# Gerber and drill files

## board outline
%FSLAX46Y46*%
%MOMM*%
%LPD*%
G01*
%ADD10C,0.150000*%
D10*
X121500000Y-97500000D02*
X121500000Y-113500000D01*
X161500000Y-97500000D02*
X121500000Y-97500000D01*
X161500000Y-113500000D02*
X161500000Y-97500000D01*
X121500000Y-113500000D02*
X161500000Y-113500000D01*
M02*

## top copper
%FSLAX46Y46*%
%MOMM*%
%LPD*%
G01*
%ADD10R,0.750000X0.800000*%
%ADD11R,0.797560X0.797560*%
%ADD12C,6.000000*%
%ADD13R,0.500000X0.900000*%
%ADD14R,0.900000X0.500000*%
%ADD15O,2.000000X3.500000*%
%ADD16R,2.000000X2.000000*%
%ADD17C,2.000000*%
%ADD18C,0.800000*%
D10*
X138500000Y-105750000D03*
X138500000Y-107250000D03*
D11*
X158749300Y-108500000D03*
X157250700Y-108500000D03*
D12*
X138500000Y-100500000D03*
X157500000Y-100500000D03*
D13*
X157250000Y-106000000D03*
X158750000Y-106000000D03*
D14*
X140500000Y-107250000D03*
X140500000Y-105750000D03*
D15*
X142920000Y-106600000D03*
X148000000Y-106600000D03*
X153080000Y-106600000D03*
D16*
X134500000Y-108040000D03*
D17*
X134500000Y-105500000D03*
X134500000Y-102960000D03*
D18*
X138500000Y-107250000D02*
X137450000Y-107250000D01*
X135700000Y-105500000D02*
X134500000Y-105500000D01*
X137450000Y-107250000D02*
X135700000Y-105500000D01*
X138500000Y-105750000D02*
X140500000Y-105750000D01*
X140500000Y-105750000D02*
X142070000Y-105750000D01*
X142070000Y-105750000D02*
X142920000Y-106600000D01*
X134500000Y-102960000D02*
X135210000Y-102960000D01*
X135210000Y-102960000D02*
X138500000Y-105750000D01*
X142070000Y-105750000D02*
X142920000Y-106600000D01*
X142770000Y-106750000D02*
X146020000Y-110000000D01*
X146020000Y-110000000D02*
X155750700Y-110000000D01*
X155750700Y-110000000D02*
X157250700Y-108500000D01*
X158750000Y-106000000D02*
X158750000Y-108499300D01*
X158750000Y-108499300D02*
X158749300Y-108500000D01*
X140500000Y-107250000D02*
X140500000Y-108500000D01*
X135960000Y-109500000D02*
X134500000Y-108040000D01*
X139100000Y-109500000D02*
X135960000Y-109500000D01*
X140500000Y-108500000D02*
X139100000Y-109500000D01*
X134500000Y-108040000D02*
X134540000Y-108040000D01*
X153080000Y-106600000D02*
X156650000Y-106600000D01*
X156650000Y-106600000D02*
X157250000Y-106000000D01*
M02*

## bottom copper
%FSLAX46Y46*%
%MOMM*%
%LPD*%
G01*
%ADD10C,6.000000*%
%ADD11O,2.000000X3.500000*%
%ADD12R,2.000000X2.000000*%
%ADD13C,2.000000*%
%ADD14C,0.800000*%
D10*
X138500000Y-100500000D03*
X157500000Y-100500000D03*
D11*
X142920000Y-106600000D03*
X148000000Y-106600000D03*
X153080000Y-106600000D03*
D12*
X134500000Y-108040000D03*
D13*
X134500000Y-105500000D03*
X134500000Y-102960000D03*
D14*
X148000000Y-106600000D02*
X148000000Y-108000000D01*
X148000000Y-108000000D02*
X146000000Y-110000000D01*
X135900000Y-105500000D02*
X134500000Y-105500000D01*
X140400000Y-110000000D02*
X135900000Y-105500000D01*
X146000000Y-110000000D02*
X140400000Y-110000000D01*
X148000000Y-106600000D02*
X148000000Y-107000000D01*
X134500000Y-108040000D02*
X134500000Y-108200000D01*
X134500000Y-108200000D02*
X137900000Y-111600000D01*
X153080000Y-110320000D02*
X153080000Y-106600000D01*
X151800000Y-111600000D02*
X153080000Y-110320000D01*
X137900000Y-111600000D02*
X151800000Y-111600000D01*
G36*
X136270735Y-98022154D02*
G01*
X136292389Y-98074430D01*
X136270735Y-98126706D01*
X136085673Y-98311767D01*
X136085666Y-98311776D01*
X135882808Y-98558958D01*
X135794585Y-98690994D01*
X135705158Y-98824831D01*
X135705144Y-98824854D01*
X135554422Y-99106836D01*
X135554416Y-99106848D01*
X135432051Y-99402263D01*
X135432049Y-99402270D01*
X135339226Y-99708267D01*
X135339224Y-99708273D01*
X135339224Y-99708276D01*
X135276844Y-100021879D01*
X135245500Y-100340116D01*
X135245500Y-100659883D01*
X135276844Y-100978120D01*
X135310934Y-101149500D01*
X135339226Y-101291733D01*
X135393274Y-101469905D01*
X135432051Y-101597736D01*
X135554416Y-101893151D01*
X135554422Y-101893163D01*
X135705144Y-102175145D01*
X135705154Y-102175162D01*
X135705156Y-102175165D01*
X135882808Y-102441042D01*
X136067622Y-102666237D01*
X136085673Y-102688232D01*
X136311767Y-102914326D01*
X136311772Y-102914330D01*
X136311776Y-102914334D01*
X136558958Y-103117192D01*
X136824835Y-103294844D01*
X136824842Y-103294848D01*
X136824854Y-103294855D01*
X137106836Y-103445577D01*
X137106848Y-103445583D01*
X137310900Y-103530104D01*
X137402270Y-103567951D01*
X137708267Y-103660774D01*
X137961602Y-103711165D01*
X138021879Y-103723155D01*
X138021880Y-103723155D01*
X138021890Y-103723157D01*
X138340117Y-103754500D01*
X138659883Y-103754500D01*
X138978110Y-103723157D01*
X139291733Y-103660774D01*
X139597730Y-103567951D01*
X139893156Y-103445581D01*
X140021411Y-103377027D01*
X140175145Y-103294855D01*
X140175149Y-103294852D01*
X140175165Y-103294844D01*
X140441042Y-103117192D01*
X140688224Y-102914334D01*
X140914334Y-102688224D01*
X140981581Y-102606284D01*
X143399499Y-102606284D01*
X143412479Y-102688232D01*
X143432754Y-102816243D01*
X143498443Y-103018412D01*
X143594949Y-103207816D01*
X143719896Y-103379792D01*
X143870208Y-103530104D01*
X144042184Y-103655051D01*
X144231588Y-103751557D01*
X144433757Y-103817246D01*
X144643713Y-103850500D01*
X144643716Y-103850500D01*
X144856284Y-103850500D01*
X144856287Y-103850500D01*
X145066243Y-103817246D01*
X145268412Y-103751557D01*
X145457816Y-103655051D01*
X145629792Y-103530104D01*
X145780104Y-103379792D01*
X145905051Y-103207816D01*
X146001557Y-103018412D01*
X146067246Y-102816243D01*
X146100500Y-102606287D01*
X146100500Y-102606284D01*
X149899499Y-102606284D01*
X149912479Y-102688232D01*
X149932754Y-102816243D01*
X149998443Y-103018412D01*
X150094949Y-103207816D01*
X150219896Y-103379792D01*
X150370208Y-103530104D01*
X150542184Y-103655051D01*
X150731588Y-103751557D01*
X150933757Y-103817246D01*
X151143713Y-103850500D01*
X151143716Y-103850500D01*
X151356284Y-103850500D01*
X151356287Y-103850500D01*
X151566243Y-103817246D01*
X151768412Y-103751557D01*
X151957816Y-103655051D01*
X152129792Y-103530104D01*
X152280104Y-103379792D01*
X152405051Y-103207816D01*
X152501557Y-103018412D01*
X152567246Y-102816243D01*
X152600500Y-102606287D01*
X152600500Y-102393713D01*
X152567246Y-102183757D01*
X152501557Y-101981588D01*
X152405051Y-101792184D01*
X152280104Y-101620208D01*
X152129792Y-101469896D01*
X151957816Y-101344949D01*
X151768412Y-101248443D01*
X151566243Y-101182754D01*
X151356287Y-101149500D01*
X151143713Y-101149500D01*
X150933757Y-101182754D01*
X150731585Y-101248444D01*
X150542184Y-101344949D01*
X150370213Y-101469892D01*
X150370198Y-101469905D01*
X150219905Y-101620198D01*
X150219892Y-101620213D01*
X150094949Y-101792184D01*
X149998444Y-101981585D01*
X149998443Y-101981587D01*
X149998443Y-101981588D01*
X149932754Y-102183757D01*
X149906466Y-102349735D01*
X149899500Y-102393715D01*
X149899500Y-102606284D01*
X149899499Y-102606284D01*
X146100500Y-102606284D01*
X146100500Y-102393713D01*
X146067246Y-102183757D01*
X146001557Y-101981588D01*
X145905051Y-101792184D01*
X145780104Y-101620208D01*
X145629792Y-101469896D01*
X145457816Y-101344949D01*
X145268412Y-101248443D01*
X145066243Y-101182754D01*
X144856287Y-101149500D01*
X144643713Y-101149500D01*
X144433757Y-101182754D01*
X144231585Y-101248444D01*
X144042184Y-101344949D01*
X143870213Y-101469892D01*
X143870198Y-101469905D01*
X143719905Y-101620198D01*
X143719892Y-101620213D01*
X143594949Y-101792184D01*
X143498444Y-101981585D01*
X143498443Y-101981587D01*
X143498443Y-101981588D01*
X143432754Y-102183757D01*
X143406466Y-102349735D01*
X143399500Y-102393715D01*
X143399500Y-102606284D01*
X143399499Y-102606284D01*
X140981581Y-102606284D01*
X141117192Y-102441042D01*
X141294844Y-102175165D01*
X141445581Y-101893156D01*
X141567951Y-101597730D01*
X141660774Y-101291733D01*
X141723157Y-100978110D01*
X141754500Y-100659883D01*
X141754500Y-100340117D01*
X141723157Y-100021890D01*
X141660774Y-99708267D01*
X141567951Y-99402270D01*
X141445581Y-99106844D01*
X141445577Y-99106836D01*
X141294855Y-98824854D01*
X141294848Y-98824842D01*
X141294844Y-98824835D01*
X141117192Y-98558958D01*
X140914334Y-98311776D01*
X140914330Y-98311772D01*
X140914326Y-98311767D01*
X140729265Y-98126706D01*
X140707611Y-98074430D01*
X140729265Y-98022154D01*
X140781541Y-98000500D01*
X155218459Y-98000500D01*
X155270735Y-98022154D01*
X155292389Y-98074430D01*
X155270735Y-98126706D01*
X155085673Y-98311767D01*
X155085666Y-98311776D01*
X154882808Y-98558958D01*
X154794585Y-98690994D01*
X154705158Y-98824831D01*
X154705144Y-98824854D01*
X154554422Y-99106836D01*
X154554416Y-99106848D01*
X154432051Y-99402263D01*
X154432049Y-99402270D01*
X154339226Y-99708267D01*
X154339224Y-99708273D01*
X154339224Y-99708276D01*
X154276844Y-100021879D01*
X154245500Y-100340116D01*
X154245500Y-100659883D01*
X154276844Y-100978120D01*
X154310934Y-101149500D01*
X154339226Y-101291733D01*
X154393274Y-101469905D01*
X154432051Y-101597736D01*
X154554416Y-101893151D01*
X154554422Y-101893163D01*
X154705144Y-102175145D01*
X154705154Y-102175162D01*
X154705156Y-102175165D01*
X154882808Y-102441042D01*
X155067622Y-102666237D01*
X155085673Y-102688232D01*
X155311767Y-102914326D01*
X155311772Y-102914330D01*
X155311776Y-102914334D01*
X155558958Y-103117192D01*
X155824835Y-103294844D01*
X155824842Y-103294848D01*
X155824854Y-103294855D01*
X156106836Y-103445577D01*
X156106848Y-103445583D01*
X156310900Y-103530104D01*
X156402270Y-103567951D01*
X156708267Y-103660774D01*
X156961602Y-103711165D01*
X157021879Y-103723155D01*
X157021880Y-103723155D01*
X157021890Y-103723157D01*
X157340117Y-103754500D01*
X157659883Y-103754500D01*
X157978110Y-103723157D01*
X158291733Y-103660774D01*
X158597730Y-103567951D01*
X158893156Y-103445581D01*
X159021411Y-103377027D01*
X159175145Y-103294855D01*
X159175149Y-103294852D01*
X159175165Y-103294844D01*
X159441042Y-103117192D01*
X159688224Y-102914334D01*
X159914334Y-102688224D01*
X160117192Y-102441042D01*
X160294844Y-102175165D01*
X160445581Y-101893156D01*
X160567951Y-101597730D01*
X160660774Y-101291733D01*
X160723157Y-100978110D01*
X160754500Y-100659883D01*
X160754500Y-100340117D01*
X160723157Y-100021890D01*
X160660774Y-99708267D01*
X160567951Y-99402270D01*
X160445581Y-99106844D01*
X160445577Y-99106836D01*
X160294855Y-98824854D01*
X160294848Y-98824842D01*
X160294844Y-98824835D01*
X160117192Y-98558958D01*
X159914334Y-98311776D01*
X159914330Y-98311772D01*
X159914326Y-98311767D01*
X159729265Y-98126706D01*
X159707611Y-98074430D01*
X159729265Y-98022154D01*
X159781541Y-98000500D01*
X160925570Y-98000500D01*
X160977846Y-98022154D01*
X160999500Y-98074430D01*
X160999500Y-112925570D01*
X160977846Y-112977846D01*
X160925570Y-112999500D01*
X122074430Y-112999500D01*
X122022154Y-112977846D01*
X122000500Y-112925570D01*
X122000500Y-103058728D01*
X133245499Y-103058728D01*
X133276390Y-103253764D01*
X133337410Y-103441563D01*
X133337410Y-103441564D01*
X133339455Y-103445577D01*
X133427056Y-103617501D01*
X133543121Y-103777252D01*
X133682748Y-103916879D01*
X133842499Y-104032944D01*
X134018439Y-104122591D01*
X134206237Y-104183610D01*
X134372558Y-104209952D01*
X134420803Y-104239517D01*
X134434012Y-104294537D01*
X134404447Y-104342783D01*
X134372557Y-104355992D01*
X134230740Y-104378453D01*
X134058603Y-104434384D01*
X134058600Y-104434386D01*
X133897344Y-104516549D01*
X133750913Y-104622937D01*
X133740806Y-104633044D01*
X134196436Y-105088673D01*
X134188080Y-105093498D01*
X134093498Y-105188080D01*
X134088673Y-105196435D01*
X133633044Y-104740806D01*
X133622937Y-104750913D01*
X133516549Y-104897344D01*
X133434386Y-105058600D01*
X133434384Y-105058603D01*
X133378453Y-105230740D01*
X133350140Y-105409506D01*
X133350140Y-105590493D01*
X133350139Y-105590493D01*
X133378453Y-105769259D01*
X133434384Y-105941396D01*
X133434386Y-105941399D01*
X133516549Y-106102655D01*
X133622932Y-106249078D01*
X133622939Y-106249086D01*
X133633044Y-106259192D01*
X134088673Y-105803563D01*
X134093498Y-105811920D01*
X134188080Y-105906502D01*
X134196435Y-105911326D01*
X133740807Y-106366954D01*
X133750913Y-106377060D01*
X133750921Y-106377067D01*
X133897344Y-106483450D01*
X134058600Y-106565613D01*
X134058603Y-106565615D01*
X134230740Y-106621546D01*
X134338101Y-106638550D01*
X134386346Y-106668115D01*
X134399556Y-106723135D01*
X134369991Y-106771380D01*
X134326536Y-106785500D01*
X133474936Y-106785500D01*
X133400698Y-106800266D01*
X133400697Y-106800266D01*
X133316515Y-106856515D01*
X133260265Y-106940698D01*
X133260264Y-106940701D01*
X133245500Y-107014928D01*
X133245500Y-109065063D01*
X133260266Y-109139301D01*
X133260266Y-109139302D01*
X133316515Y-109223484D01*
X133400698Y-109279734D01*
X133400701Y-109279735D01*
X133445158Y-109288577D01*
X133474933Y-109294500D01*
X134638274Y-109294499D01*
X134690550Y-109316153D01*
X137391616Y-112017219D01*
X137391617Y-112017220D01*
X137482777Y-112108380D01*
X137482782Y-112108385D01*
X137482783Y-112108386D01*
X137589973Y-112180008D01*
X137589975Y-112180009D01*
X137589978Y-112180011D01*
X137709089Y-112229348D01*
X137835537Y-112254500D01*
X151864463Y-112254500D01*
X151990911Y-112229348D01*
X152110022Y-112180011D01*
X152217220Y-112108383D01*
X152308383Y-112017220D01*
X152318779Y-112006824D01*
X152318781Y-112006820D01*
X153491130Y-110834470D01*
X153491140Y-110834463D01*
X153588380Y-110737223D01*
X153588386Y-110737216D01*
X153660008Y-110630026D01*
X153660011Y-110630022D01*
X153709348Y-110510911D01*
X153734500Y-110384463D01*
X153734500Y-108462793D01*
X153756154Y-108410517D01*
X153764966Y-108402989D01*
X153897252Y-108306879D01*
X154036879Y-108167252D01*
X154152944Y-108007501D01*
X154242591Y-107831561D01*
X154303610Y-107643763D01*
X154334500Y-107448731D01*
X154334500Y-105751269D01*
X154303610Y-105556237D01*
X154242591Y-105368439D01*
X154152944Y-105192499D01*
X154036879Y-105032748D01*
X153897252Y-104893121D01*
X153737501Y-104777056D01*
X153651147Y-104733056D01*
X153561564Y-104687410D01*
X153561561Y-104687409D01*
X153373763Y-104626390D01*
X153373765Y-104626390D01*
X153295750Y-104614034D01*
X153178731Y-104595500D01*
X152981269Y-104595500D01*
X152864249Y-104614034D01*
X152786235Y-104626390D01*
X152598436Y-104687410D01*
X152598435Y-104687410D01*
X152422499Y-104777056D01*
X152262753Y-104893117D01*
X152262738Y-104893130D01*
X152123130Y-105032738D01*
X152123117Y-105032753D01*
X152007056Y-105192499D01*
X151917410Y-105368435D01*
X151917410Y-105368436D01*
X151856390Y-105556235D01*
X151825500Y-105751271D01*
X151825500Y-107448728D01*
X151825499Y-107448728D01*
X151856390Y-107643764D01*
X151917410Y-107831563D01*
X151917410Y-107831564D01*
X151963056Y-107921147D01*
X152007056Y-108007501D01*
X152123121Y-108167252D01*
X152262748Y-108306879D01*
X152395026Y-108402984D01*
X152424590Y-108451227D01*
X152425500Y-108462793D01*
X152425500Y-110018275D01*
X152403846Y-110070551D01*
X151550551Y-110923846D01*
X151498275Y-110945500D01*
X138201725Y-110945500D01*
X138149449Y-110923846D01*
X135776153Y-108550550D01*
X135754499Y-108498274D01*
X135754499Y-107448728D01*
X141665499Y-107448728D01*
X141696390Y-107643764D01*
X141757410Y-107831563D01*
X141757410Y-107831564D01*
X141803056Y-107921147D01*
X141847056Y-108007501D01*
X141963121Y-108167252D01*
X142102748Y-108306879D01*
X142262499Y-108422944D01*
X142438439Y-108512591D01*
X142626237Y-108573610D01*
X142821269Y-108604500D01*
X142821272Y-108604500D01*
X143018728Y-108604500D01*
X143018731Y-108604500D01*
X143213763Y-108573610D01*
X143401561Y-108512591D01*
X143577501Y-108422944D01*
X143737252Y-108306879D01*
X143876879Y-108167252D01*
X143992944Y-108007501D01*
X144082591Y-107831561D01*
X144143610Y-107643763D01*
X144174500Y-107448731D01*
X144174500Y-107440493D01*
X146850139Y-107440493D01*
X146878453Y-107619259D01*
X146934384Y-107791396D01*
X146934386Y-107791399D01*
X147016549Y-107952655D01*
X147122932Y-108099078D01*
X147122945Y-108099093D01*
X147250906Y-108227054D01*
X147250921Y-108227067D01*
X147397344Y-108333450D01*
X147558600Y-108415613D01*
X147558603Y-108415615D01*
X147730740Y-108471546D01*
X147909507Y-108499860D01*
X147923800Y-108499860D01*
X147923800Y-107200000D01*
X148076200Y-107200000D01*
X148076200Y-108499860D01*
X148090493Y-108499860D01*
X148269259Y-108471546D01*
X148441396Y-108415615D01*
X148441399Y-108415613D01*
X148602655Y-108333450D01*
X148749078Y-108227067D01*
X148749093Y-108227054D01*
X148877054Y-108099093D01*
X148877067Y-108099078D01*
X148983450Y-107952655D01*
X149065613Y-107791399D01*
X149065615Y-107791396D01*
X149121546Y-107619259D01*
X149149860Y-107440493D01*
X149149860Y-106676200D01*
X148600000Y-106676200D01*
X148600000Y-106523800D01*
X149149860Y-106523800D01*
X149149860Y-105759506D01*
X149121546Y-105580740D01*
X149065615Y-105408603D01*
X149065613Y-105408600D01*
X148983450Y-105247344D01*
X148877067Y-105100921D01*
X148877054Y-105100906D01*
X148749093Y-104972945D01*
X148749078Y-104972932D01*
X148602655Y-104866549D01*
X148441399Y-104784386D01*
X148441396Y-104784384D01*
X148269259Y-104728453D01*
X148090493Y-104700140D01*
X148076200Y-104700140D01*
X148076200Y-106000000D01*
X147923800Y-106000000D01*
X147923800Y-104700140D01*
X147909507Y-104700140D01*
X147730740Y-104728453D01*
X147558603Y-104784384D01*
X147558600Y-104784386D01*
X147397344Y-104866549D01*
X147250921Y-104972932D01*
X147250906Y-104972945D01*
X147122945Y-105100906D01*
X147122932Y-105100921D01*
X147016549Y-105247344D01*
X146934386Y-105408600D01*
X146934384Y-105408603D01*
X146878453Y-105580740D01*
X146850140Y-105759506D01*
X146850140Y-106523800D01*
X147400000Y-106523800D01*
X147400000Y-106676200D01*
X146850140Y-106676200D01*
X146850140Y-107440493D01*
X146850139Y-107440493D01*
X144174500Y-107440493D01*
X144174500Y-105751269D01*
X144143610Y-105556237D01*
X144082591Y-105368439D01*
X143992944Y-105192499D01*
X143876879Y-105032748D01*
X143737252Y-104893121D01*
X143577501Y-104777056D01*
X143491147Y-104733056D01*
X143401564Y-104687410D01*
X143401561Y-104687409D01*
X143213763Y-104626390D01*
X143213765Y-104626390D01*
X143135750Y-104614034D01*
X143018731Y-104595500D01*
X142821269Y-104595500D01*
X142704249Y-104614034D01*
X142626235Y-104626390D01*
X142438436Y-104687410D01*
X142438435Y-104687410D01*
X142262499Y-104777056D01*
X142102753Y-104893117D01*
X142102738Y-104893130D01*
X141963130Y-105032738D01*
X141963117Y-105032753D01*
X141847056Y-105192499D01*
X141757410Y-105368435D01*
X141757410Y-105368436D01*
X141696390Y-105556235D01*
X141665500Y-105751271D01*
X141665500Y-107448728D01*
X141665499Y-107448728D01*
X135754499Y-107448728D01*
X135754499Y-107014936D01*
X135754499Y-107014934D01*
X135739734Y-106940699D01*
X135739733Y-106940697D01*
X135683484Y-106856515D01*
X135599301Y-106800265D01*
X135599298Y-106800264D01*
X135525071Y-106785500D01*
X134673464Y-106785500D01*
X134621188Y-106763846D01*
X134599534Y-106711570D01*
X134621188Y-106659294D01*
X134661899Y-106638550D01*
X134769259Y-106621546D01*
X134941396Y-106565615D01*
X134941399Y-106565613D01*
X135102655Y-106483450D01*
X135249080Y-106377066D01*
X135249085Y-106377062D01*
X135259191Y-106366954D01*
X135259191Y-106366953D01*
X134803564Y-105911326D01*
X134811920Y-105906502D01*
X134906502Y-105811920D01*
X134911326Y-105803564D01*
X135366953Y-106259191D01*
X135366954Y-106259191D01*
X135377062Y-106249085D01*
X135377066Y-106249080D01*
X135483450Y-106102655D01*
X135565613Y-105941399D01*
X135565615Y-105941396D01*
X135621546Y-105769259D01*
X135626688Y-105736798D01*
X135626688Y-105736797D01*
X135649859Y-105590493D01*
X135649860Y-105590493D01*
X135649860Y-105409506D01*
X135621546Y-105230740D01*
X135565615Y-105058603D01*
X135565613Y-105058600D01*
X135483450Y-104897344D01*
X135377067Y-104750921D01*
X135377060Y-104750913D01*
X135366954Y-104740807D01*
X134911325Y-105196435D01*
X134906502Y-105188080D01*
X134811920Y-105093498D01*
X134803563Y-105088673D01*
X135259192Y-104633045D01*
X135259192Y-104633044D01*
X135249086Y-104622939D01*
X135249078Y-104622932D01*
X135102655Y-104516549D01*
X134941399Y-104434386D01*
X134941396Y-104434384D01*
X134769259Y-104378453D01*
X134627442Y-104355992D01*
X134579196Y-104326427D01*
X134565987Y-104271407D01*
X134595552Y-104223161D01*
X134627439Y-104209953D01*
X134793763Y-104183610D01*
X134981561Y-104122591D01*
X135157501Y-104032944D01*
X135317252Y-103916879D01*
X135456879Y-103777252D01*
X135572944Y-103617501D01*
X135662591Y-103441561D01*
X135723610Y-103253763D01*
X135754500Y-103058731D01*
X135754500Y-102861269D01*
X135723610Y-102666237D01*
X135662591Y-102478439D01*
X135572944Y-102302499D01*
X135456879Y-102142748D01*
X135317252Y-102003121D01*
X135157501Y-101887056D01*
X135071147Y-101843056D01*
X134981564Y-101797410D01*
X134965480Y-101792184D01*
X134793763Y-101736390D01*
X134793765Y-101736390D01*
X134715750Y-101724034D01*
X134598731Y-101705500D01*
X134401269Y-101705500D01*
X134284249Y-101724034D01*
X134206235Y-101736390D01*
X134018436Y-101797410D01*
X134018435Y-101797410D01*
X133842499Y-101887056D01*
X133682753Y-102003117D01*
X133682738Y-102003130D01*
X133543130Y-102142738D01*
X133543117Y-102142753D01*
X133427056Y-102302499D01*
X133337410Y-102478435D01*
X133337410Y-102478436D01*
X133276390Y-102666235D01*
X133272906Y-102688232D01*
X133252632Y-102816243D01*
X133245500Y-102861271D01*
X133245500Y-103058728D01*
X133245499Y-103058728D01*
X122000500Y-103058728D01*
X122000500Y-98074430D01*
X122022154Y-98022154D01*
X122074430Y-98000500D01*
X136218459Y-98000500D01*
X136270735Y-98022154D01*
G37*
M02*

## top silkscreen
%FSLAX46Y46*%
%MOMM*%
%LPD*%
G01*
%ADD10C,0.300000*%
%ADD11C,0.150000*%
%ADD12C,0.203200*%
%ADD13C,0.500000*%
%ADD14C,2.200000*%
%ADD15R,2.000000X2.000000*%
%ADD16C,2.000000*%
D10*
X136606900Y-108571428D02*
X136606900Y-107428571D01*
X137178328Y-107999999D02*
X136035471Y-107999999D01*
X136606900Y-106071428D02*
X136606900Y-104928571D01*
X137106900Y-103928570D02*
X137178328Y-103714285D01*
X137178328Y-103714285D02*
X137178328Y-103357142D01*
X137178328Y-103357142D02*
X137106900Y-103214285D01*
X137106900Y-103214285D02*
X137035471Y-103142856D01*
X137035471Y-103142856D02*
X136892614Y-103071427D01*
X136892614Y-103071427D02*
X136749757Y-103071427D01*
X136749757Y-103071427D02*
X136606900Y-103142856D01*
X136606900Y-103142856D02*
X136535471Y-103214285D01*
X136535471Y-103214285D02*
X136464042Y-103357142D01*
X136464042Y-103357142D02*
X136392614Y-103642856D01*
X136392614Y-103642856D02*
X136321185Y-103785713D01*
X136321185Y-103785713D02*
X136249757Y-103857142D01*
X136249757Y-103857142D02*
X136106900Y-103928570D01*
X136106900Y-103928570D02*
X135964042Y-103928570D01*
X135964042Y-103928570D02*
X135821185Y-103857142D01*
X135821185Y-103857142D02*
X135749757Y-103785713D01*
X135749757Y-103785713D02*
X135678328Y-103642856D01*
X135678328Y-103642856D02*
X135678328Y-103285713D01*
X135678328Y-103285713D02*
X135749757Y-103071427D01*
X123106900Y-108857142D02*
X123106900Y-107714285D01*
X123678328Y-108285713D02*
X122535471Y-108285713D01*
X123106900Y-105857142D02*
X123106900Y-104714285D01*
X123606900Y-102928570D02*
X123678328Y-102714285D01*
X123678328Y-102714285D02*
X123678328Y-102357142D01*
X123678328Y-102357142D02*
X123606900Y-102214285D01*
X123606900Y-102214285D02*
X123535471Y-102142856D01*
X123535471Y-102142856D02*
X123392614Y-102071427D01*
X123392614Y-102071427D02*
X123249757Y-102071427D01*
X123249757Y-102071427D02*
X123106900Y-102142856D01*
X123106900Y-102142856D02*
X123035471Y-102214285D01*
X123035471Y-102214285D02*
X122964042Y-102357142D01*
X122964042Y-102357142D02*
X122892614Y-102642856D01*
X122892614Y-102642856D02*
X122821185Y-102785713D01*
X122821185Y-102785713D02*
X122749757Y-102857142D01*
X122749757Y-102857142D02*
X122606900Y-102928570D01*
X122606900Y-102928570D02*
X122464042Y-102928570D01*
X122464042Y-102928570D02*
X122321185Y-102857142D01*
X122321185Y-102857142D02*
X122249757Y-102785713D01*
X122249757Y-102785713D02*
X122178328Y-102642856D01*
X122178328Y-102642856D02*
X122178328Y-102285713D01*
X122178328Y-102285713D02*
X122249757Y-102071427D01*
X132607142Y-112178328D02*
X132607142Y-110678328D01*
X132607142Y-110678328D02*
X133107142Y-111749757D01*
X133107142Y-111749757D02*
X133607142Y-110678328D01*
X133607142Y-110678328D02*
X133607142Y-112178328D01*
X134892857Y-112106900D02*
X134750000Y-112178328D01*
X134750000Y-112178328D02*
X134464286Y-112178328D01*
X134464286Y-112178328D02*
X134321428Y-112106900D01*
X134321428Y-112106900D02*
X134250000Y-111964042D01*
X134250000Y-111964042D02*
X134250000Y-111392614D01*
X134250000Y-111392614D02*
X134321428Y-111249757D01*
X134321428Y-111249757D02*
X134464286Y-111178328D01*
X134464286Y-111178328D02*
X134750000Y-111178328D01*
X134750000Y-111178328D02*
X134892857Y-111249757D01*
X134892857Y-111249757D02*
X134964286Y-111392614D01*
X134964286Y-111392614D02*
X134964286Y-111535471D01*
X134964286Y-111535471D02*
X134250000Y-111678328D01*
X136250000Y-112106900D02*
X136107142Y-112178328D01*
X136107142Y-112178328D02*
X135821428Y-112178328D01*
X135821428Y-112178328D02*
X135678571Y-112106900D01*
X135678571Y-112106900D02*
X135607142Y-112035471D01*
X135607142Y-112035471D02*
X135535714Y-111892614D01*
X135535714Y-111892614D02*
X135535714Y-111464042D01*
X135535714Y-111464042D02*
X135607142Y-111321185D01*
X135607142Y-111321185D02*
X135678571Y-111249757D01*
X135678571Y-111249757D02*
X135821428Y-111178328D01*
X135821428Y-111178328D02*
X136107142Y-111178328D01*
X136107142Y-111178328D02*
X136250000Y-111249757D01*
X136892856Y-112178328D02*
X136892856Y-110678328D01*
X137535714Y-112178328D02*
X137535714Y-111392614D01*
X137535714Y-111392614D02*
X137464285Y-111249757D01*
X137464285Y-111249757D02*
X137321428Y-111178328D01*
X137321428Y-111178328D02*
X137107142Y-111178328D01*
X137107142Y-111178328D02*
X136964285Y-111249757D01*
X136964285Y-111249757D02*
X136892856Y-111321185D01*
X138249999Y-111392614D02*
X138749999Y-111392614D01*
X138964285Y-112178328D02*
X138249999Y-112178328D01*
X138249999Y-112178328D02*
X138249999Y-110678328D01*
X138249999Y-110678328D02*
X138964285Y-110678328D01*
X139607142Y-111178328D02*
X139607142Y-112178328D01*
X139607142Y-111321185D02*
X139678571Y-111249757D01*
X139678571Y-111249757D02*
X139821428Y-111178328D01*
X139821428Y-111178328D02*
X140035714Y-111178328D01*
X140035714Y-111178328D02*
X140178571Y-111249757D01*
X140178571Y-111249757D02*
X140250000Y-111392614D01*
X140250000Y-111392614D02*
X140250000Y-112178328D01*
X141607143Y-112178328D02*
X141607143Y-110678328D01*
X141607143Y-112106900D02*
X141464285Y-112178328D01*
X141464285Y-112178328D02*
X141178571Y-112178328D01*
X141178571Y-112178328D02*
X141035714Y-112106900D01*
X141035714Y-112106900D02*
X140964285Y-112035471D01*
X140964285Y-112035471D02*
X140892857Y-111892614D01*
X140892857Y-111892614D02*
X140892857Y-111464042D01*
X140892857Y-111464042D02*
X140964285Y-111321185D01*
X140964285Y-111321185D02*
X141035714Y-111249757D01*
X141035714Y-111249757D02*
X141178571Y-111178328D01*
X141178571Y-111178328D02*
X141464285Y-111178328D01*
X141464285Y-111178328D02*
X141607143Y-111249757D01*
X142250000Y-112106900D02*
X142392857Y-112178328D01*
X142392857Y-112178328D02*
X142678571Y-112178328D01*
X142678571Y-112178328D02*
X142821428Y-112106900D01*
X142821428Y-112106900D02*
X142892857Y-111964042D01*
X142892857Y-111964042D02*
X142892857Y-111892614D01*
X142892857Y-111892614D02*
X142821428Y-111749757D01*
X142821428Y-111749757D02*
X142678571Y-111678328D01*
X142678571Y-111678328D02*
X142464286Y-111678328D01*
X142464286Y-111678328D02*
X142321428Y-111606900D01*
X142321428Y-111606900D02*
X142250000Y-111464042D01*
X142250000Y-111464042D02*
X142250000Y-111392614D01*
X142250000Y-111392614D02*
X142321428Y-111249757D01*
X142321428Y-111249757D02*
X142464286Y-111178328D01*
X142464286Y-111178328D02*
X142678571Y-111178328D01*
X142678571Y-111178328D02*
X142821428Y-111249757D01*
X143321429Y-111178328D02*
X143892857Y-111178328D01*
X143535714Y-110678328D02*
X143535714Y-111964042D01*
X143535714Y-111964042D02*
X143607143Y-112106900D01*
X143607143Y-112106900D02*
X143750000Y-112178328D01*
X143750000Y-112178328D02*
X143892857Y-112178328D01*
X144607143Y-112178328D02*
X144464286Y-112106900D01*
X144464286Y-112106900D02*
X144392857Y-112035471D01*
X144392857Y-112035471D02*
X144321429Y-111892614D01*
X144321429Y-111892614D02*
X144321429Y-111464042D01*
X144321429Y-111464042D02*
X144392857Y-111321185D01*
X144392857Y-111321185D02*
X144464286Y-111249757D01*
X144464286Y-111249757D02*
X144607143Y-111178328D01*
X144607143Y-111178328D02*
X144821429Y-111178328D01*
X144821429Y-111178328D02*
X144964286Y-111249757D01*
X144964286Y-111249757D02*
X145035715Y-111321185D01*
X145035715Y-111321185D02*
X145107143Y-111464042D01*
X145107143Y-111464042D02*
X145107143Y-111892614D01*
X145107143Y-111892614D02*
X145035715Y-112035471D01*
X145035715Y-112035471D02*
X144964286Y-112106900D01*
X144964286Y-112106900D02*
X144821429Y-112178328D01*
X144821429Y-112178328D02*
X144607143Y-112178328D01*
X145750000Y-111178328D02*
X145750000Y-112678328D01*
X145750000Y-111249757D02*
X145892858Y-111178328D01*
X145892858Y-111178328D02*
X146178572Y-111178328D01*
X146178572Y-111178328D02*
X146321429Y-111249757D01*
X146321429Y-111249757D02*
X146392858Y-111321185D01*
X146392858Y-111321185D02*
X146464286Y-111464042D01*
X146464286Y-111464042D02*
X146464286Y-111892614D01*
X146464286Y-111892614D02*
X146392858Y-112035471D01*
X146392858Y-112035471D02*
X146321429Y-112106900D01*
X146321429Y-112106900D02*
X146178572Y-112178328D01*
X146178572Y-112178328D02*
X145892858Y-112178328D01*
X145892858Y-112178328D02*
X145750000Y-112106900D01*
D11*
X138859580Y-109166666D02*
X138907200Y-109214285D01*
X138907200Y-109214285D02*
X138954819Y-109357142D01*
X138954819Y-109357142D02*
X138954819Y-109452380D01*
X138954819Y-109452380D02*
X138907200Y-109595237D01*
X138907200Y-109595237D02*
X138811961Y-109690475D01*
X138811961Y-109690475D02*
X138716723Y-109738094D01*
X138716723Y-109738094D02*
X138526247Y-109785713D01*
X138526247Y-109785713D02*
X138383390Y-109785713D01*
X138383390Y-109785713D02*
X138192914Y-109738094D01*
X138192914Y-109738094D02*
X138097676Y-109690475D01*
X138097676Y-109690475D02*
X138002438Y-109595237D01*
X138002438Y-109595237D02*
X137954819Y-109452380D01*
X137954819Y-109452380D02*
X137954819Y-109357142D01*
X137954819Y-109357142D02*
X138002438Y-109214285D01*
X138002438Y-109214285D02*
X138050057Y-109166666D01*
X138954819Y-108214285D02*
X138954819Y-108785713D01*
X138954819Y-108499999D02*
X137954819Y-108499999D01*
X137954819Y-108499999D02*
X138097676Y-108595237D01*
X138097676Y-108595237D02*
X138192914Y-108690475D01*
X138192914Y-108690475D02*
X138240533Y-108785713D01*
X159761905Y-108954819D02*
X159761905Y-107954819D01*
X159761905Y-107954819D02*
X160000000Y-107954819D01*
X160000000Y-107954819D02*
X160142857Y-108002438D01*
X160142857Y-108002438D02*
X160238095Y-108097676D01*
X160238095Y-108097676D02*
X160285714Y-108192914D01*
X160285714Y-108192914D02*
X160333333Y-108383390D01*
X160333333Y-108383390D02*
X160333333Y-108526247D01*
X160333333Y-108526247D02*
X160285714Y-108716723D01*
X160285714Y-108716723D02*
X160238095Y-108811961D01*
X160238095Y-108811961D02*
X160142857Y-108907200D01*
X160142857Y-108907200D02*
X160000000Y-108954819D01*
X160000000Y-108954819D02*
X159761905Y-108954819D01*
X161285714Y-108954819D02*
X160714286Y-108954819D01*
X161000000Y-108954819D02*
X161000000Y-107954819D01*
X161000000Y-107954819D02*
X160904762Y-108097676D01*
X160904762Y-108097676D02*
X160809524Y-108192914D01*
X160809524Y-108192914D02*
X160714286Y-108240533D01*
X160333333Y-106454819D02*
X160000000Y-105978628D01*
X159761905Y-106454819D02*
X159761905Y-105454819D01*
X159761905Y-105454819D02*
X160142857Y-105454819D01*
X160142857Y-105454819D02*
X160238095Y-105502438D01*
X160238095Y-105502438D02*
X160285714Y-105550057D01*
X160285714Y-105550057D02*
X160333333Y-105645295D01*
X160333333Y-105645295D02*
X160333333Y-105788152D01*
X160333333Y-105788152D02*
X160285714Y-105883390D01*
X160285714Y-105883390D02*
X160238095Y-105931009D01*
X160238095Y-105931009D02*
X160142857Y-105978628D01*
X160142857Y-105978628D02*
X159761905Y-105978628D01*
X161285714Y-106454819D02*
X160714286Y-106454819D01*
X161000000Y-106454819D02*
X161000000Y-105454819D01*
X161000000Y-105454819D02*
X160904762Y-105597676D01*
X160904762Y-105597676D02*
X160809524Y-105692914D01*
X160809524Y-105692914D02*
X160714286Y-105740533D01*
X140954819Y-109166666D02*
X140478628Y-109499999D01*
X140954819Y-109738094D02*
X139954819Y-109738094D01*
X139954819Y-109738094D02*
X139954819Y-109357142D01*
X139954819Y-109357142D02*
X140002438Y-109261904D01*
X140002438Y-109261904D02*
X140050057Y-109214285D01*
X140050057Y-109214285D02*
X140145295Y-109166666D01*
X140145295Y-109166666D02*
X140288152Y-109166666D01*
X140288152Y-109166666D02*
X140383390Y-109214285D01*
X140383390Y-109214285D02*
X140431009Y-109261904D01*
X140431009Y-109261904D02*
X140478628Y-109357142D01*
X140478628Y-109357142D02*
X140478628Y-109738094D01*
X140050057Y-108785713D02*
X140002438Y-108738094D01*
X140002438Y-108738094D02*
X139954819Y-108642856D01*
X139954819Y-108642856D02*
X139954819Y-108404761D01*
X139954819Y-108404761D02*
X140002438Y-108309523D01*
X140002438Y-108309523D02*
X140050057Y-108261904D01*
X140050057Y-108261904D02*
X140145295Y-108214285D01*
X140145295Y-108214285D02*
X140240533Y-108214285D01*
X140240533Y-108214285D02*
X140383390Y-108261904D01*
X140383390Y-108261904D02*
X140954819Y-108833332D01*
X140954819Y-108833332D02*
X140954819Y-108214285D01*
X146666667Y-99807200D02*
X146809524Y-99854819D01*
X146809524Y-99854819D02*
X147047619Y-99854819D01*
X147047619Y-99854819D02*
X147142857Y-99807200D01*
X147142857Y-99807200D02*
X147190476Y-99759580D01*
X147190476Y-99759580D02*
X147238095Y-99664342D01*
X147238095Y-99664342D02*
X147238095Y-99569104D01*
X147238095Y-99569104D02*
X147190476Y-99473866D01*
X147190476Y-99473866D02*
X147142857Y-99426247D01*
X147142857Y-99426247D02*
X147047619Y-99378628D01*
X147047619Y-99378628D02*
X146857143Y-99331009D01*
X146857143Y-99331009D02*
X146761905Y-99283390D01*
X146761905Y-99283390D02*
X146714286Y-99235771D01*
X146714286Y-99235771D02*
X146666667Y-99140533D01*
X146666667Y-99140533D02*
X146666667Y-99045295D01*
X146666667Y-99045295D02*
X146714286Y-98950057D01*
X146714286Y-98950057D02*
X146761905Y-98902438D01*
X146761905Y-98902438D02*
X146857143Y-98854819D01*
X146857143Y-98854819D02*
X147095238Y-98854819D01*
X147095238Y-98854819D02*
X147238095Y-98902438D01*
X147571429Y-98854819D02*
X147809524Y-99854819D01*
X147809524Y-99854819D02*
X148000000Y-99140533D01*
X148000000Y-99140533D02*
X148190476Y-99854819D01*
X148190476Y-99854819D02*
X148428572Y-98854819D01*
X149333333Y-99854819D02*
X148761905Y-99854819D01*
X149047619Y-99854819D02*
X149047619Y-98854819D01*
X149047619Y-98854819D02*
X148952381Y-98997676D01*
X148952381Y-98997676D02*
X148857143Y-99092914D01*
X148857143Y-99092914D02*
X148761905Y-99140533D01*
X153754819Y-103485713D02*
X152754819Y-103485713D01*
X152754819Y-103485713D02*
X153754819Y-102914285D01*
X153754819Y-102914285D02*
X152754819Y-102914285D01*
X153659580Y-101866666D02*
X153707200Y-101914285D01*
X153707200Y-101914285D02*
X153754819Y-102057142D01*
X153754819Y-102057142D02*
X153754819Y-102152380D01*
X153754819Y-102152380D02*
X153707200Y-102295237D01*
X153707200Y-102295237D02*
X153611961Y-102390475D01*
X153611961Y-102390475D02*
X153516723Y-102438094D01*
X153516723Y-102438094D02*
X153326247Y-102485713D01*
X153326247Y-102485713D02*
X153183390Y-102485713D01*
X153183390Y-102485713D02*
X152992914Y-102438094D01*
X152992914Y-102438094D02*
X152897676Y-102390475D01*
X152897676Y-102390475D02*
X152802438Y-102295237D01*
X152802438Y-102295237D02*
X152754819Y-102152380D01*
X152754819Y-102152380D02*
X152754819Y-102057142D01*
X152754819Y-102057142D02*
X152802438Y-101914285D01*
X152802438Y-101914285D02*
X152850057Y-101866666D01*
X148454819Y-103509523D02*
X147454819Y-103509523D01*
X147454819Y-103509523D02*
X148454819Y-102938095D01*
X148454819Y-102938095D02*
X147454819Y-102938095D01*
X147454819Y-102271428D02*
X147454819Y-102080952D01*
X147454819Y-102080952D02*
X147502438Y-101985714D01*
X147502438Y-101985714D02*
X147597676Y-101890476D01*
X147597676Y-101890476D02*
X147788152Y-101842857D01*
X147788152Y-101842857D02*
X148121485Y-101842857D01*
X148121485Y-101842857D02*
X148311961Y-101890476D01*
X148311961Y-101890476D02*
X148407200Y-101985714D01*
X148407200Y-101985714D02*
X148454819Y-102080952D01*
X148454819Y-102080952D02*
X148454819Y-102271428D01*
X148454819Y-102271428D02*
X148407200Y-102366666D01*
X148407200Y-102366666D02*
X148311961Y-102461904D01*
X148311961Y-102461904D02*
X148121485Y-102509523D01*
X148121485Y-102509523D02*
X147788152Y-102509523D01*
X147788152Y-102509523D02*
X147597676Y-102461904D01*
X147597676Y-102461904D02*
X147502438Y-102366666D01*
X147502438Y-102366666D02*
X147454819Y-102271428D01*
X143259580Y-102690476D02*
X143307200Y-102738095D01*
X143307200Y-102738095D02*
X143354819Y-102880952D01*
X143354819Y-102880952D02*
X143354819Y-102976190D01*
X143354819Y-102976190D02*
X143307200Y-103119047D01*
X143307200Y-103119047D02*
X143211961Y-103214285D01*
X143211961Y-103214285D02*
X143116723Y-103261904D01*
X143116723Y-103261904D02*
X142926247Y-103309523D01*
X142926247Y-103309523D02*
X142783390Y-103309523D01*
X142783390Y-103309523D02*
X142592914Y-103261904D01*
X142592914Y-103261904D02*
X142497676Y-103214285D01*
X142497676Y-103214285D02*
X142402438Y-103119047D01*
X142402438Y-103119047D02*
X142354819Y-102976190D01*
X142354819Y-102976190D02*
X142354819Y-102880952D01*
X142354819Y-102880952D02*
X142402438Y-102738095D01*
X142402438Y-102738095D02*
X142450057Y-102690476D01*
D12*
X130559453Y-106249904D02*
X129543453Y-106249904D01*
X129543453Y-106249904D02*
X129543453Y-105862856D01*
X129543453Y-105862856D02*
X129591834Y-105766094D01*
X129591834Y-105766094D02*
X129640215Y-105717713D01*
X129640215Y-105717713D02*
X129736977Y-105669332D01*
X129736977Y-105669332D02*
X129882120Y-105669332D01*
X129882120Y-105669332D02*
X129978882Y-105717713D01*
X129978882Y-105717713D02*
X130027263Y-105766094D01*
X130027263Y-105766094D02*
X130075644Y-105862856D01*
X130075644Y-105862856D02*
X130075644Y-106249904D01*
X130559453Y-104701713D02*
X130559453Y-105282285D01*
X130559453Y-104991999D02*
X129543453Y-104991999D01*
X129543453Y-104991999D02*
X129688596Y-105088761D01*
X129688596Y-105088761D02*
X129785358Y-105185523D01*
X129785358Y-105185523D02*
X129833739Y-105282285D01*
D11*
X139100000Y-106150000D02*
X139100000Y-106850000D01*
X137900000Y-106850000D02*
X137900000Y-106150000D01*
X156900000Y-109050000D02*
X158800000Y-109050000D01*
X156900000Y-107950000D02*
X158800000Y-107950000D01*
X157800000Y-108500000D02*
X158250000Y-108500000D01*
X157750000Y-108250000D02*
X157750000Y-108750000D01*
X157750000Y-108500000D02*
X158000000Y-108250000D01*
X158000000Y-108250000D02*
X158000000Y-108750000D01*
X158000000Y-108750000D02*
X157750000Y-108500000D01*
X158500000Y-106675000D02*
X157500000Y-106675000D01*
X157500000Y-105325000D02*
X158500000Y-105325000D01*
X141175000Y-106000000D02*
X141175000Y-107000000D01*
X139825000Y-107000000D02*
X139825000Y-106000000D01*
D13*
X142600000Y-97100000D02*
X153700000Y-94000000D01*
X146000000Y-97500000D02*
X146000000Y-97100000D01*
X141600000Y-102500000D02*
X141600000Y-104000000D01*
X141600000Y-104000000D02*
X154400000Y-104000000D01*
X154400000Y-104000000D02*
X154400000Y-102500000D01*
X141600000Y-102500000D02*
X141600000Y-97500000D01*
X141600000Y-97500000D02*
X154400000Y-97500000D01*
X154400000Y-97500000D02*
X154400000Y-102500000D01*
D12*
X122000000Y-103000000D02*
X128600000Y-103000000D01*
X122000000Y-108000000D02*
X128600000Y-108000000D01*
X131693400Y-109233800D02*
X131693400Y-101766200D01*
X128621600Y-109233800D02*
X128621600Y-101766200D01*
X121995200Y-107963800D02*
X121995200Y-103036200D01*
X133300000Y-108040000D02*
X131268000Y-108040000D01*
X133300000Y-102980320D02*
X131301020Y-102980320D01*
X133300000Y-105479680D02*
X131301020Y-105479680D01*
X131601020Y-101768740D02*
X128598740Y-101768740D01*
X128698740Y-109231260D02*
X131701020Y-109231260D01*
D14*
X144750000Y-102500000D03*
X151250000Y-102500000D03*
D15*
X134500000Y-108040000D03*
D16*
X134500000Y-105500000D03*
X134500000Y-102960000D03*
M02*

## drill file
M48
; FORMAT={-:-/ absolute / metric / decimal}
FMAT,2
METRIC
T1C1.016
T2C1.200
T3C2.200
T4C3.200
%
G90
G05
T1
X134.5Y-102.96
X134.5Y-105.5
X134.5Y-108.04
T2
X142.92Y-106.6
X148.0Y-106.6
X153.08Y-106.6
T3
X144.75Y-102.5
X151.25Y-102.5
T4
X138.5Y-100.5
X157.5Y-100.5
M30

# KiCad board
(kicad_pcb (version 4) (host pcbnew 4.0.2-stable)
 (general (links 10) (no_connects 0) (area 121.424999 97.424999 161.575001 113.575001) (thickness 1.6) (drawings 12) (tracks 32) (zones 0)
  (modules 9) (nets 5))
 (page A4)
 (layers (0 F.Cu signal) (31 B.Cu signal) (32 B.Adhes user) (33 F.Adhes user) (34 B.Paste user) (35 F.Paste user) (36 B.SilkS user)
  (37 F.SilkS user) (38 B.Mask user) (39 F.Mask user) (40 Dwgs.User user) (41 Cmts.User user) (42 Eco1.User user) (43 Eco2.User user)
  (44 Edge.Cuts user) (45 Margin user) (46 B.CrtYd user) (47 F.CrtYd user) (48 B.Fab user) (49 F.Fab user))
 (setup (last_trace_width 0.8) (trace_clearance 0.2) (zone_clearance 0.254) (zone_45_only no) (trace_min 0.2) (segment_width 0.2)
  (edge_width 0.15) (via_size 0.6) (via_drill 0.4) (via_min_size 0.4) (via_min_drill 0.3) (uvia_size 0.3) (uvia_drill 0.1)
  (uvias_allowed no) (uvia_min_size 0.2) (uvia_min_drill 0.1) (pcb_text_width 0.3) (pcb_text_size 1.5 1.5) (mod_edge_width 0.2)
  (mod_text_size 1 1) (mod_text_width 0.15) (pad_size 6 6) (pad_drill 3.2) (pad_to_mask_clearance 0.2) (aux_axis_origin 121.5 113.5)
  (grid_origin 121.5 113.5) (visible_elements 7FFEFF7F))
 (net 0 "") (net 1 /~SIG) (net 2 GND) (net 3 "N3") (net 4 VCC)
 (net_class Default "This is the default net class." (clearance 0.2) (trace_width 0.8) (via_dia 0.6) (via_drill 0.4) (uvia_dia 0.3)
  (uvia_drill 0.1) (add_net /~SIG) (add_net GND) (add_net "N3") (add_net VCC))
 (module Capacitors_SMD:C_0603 (layer F.Cu) (at 138.5 106.5 270)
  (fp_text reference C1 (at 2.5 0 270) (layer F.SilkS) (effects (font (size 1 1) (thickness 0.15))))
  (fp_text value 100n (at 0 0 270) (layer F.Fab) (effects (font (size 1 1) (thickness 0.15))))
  (fp_line (start -0.35 -0.6) (end 0.35 -0.6) (layer F.SilkS) (width 0.15))
  (fp_line (start 0.35 0.6) (end -0.35 0.6) (layer F.SilkS) (width 0.15))
  (pad 1 smd rect (at -0.75 0 270) (size 0.8 0.75) (layers F.Cu F.Paste F.Mask) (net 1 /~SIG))
  (pad 2 smd rect (at 0.75 0 270) (size 0.8 0.75) (layers F.Cu F.Paste F.Mask) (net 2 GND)))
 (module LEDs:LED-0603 (layer F.Cu) (at 158 108.5)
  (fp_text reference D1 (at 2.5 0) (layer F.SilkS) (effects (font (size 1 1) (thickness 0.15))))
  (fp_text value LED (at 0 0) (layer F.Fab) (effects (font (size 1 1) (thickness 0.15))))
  (fp_line (start -1.1 0.55) (end 0.8 0.55) (layer F.SilkS) (width 0.15))
  (fp_line (start -1.1 -0.55) (end 0.8 -0.55) (layer F.SilkS) (width 0.15))
  (fp_line (start -0.2 0) (end 0.25 0) (layer F.SilkS) (width 0.15))
  (fp_line (start -0.25 -0.25) (end -0.25 0.25) (layer F.SilkS) (width 0.15))
  (fp_line (start -0.25 0) (end 0 -0.25) (layer F.SilkS) (width 0.15))
  (fp_line (start 0 -0.25) (end 0 0.25) (layer F.SilkS) (width 0.15))
  (fp_line (start 0 0.25) (end -0.25 0) (layer F.SilkS) (width 0.15))
  (pad 2 smd rect (at 0.7493 0 180) (size 0.79756 0.79756) (layers F.Cu F.Paste F.Mask) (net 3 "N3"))
  (pad 1 smd rect (at -0.7493 0 180) (size 0.79756 0.79756) (layers F.Cu F.Paste F.Mask) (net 1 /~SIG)))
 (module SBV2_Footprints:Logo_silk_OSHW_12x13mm (layer B.Cu) (at 127.5 104 180)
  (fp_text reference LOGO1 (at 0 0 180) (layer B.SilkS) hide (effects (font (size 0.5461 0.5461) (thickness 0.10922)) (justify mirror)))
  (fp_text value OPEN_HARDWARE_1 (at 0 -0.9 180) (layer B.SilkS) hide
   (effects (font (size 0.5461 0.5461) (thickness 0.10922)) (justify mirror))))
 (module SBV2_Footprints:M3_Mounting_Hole (layer F.Cu) (at 138.5 100.5)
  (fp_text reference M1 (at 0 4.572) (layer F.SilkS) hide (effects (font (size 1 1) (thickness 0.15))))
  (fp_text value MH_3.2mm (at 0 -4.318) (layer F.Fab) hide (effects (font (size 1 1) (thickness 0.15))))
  (pad "" np_thru_hole circle (at 0 0) (size 6 6) (drill 3.2) (layers *.Cu *.Mask)))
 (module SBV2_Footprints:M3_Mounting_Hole (layer F.Cu) (at 157.5 100.5)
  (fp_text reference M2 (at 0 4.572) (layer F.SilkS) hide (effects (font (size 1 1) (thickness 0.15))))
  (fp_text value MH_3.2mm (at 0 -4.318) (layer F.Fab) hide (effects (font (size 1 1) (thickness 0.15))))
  (pad "" np_thru_hole circle (at 0 0) (size 6 6) (drill 3.2) (layers *.Cu *.Mask)))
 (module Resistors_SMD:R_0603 (layer F.Cu) (at 158 106)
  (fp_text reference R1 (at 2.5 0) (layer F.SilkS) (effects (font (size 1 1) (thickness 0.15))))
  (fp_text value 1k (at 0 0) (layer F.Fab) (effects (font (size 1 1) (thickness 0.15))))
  (fp_line (start 0.5 0.675) (end -0.5 0.675) (layer F.SilkS) (width 0.15))
  (fp_line (start -0.5 -0.675) (end 0.5 -0.675) (layer F.SilkS) (width 0.15))
  (pad 1 smd rect (at -0.75 0) (size 0.5 0.9) (layers F.Cu F.Paste F.Mask) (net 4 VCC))
  (pad 2 smd rect (at 0.75 0) (size 0.5 0.9) (layers F.Cu F.Paste F.Mask) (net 3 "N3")))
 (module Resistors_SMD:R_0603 (layer F.Cu) (at 140.5 106.5 90)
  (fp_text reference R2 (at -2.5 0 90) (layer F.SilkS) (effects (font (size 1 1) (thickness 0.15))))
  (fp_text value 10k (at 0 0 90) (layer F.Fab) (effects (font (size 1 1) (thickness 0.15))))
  (fp_line (start 0.5 0.675) (end -0.5 0.675) (layer F.SilkS) (width 0.15))
  (fp_line (start -0.5 -0.675) (end 0.5 -0.675) (layer F.SilkS) (width 0.15))
  (pad 1 smd rect (at -0.75 0 90) (size 0.5 0.9) (layers F.Cu F.Paste F.Mask) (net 4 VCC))
  (pad 2 smd rect (at 0.75 0 90) (size 0.5 0.9) (layers F.Cu F.Paste F.Mask) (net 1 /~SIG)))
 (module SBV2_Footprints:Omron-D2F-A (layer F.Cu) (at 148 102.5)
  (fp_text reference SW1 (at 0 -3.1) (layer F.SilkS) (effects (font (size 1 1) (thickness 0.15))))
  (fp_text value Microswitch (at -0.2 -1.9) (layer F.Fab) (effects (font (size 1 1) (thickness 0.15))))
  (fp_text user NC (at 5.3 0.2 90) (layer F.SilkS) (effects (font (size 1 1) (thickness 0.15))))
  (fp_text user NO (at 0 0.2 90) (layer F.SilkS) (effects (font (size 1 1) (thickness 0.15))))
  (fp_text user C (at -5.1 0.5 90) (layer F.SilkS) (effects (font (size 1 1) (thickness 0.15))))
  (fp_line (start -5.4 -5.4) (end 5.7 -8.5) (layer F.SilkS) (width 0.5))
  (fp_line (start -2 -5) (end -2 -5.4) (layer F.SilkS) (width 0.5))
  (fp_line (start -6.4 0) (end -6.4 1.5) (layer F.SilkS) (width 0.5))
  (fp_line (start -6.4 1.5) (end 6.4 1.5) (layer F.SilkS) (width 0.5))
  (fp_line (start 6.4 1.5) (end 6.4 0) (layer F.SilkS) (width 0.5))
  (fp_line (start -6.4 0) (end -6.4 -5) (layer F.SilkS) (width 0.5))
  (fp_line (start -6.4 -5) (end 6.4 -5) (layer F.SilkS) (width 0.5))
  (fp_line (start 6.4 -5) (end 6.4 0) (layer F.SilkS) (width 0.5))
  (pad "" np_thru_hole circle (at -3.25 0) (size 2.2 2.2) (drill 2.2) (layers *.Cu *.Mask F.SilkS))
  (pad "" np_thru_hole circle (at 3.25 0) (size 2.2 2.2) (drill 2.2) (layers *.Cu *.Mask F.SilkS))
  (pad 1 thru_hole oval (at -5.08 4.1) (size 2 3.5) (drill 1.2) (layers *.Cu *.Mask) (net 1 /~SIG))
  (pad 2 thru_hole oval (at 0 4.1) (size 2 3.5) (drill 1.2) (layers *.Cu *.Mask) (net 2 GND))
  (pad 3 thru_hole oval (at 5.08 4.1) (size 2 3.5) (drill 1.2) (layers *.Cu *.Mask) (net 4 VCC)))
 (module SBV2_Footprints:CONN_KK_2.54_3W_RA (layer F.Cu) (at 134.5 105.5 90)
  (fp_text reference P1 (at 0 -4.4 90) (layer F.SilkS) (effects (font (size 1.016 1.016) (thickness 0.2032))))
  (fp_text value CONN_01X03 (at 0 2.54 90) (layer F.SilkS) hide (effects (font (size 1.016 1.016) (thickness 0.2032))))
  (fp_line (start 2.5 -12.5) (end 2.5 -5.9) (layer F.SilkS) (width 0.2032))
  (fp_line (start -2.5 -12.5) (end -2.5 -5.9) (layer F.SilkS) (width 0.2032))
  (fp_line (start -3.7338 -2.8066) (end 3.7338 -2.8066) (layer F.SilkS) (width 0.2032))
  (fp_line (start -3.7338 -5.8784) (end 3.7338 -5.8784) (layer F.SilkS) (width 0.2032))
  (fp_line (start -2.4638 -12.5048) (end 2.4638 -12.5048) (layer F.SilkS) (width 0.2032))
  (fp_line (start -2.54 -1.2) (end -2.54 -3.232) (layer F.SilkS) (width 0.2032))
  (fp_line (start 2.51968 -1.2) (end 2.51968 -3.19898) (layer F.SilkS) (width 0.2032))
  (fp_line (start 0.02032 -1.2) (end 0.02032 -3.19898) (layer F.SilkS) (width 0.2032))
  (fp_line (start 3.73126 -2.89898) (end 3.73126 -5.90126) (layer F.SilkS) (width 0.2032))
  (fp_line (start -3.73126 -5.80126) (end -3.73126 -2.79898) (layer F.SilkS) (width 0.2032))
  (pad 1 thru_hole rect (at -2.54 0 90) (size 2 2) (drill 1.016) (layers *.Cu *.Mask F.SilkS) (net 4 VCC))
  (pad 2 thru_hole circle (at 0 0 90) (size 2 2) (drill 1.016) (layers *.Cu *.Mask F.SilkS) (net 2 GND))
  (pad 3 thru_hole circle (at 2.54 0 90) (size 2 2) (drill 1.016) (layers *.Cu *.Mask F.SilkS) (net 1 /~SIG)))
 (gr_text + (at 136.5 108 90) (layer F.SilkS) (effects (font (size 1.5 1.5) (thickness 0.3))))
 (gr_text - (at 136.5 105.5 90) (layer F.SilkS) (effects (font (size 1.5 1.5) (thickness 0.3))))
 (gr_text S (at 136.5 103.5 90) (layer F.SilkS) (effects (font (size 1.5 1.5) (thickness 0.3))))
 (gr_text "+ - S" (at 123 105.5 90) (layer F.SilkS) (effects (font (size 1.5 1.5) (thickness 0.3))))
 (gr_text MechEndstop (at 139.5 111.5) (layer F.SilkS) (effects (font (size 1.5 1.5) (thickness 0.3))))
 (gr_line (start 121.5 97.5) (end 121.5 113.5) (angle 90) (layer Edge.Cuts) (width 0.15))
 (gr_line (start 161.5 97.5) (end 121.5 97.5) (angle 90) (layer Edge.Cuts) (width 0.15))
 (gr_line (start 161.5 113.5) (end 161.5 97.5) (angle 90) (layer Edge.Cuts) (width 0.15))
 (gr_line (start 121.5 113.5) (end 161.5 113.5) (angle 90) (layer Edge.Cuts) (width 0.15))
 (segment (start 148 106.6) (end 148 108) (width 0.8) (layer B.Cu) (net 2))
 (segment (start 148 108) (end 146 110) (width 0.8) (layer B.Cu) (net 2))
 (segment (start 135.9 105.5) (end 134.5 105.5) (width 0.8) (layer B.Cu) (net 2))
 (segment (start 140.4 110) (end 135.9 105.5) (width 0.8) (layer B.Cu) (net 2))
 (segment (start 146 110) (end 140.4 110) (width 0.8) (layer B.Cu) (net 2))
 (segment (start 138.5 107.25) (end 137.45 107.25) (width 0.8) (layer F.Cu) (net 2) (status 10))
 (segment (start 135.7 105.5) (end 134.5 105.5) (width 0.8) (layer F.Cu) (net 2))
 (segment (start 137.45 107.25) (end 135.7 105.5) (width 0.8) (layer F.Cu) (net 2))
 (segment (start 148 106.6) (end 148 107) (width 0.8) (layer B.Cu) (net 2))
 (segment (start 138.5 105.75) (end 140.5 105.75) (width 0.8) (layer F.Cu) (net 1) (status 10))
 (segment (start 140.5 105.75) (end 142.07 105.75) (width 0.8) (layer F.Cu) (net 1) (status 10))
 (segment (start 142.07 105.75) (end 142.92 106.6) (width 0.8) (layer F.Cu) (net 1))
 (segment (start 134.5 102.96) (end 135.21 102.96) (width 0.8) (layer F.Cu) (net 1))
 (segment (start 135.21 102.96) (end 138.5 105.75) (width 0.8) (layer F.Cu) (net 1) (status 20))
 (segment (start 142.07 105.75) (end 142.92 106.6) (width 0.8) (layer F.Cu) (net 1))
 (segment (start 142.77 106.75) (end 146.02 110) (width 0.8) (layer F.Cu) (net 1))
 (segment (start 146.02 110) (end 155.7507 110) (width 0.8) (layer F.Cu) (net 1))
 (segment (start 155.7507 110) (end 157.2507 108.5) (width 0.8) (layer F.Cu) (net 1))
 (segment (start 158.75 106) (end 158.75 108.4993) (width 0.8) (layer F.Cu) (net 3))
 (segment (start 158.75 108.4993) (end 158.7493 108.5) (width 0.8) (layer F.Cu) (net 3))
 (segment (start 134.5 108.04) (end 134.5 108.2) (width 0.8) (layer B.Cu) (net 4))
 (segment (start 134.5 108.2) (end 137.9 111.6) (width 0.8) (layer B.Cu) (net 4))
 (segment (start 153.08 110.32) (end 153.08 106.6) (width 0.8) (layer B.Cu) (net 4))
 (segment (start 151.8 111.6) (end 153.08 110.32) (width 0.8) (layer B.Cu) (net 4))
 (segment (start 137.9 111.6) (end 151.8 111.6) (width 0.8) (layer B.Cu) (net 4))
 (segment (start 140.5 107.25) (end 140.5 108.5) (width 0.8) (layer F.Cu) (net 4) (status 10))
 (segment (start 135.96 109.5) (end 134.5 108.04) (width 0.8) (layer F.Cu) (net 4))
 (segment (start 139.1 109.5) (end 135.96 109.5) (width 0.8) (layer F.Cu) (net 4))
 (segment (start 140.5 108.5) (end 139.1 109.5) (width 0.8) (layer F.Cu) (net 4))
 (segment (start 134.5 108.04) (end 134.54 108.04) (width 0.8) (layer F.Cu) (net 4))
 (segment (start 153.08 106.6) (end 156.65 106.6) (width 0.8) (layer F.Cu) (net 4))
 (segment (start 156.65 106.6) (end 157.25 106) (width 0.8) (layer F.Cu) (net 4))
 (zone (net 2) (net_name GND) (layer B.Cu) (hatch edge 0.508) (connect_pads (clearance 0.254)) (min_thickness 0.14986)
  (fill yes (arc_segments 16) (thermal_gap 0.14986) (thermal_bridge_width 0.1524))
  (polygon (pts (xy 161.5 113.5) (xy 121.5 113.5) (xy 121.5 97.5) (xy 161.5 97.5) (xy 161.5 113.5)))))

